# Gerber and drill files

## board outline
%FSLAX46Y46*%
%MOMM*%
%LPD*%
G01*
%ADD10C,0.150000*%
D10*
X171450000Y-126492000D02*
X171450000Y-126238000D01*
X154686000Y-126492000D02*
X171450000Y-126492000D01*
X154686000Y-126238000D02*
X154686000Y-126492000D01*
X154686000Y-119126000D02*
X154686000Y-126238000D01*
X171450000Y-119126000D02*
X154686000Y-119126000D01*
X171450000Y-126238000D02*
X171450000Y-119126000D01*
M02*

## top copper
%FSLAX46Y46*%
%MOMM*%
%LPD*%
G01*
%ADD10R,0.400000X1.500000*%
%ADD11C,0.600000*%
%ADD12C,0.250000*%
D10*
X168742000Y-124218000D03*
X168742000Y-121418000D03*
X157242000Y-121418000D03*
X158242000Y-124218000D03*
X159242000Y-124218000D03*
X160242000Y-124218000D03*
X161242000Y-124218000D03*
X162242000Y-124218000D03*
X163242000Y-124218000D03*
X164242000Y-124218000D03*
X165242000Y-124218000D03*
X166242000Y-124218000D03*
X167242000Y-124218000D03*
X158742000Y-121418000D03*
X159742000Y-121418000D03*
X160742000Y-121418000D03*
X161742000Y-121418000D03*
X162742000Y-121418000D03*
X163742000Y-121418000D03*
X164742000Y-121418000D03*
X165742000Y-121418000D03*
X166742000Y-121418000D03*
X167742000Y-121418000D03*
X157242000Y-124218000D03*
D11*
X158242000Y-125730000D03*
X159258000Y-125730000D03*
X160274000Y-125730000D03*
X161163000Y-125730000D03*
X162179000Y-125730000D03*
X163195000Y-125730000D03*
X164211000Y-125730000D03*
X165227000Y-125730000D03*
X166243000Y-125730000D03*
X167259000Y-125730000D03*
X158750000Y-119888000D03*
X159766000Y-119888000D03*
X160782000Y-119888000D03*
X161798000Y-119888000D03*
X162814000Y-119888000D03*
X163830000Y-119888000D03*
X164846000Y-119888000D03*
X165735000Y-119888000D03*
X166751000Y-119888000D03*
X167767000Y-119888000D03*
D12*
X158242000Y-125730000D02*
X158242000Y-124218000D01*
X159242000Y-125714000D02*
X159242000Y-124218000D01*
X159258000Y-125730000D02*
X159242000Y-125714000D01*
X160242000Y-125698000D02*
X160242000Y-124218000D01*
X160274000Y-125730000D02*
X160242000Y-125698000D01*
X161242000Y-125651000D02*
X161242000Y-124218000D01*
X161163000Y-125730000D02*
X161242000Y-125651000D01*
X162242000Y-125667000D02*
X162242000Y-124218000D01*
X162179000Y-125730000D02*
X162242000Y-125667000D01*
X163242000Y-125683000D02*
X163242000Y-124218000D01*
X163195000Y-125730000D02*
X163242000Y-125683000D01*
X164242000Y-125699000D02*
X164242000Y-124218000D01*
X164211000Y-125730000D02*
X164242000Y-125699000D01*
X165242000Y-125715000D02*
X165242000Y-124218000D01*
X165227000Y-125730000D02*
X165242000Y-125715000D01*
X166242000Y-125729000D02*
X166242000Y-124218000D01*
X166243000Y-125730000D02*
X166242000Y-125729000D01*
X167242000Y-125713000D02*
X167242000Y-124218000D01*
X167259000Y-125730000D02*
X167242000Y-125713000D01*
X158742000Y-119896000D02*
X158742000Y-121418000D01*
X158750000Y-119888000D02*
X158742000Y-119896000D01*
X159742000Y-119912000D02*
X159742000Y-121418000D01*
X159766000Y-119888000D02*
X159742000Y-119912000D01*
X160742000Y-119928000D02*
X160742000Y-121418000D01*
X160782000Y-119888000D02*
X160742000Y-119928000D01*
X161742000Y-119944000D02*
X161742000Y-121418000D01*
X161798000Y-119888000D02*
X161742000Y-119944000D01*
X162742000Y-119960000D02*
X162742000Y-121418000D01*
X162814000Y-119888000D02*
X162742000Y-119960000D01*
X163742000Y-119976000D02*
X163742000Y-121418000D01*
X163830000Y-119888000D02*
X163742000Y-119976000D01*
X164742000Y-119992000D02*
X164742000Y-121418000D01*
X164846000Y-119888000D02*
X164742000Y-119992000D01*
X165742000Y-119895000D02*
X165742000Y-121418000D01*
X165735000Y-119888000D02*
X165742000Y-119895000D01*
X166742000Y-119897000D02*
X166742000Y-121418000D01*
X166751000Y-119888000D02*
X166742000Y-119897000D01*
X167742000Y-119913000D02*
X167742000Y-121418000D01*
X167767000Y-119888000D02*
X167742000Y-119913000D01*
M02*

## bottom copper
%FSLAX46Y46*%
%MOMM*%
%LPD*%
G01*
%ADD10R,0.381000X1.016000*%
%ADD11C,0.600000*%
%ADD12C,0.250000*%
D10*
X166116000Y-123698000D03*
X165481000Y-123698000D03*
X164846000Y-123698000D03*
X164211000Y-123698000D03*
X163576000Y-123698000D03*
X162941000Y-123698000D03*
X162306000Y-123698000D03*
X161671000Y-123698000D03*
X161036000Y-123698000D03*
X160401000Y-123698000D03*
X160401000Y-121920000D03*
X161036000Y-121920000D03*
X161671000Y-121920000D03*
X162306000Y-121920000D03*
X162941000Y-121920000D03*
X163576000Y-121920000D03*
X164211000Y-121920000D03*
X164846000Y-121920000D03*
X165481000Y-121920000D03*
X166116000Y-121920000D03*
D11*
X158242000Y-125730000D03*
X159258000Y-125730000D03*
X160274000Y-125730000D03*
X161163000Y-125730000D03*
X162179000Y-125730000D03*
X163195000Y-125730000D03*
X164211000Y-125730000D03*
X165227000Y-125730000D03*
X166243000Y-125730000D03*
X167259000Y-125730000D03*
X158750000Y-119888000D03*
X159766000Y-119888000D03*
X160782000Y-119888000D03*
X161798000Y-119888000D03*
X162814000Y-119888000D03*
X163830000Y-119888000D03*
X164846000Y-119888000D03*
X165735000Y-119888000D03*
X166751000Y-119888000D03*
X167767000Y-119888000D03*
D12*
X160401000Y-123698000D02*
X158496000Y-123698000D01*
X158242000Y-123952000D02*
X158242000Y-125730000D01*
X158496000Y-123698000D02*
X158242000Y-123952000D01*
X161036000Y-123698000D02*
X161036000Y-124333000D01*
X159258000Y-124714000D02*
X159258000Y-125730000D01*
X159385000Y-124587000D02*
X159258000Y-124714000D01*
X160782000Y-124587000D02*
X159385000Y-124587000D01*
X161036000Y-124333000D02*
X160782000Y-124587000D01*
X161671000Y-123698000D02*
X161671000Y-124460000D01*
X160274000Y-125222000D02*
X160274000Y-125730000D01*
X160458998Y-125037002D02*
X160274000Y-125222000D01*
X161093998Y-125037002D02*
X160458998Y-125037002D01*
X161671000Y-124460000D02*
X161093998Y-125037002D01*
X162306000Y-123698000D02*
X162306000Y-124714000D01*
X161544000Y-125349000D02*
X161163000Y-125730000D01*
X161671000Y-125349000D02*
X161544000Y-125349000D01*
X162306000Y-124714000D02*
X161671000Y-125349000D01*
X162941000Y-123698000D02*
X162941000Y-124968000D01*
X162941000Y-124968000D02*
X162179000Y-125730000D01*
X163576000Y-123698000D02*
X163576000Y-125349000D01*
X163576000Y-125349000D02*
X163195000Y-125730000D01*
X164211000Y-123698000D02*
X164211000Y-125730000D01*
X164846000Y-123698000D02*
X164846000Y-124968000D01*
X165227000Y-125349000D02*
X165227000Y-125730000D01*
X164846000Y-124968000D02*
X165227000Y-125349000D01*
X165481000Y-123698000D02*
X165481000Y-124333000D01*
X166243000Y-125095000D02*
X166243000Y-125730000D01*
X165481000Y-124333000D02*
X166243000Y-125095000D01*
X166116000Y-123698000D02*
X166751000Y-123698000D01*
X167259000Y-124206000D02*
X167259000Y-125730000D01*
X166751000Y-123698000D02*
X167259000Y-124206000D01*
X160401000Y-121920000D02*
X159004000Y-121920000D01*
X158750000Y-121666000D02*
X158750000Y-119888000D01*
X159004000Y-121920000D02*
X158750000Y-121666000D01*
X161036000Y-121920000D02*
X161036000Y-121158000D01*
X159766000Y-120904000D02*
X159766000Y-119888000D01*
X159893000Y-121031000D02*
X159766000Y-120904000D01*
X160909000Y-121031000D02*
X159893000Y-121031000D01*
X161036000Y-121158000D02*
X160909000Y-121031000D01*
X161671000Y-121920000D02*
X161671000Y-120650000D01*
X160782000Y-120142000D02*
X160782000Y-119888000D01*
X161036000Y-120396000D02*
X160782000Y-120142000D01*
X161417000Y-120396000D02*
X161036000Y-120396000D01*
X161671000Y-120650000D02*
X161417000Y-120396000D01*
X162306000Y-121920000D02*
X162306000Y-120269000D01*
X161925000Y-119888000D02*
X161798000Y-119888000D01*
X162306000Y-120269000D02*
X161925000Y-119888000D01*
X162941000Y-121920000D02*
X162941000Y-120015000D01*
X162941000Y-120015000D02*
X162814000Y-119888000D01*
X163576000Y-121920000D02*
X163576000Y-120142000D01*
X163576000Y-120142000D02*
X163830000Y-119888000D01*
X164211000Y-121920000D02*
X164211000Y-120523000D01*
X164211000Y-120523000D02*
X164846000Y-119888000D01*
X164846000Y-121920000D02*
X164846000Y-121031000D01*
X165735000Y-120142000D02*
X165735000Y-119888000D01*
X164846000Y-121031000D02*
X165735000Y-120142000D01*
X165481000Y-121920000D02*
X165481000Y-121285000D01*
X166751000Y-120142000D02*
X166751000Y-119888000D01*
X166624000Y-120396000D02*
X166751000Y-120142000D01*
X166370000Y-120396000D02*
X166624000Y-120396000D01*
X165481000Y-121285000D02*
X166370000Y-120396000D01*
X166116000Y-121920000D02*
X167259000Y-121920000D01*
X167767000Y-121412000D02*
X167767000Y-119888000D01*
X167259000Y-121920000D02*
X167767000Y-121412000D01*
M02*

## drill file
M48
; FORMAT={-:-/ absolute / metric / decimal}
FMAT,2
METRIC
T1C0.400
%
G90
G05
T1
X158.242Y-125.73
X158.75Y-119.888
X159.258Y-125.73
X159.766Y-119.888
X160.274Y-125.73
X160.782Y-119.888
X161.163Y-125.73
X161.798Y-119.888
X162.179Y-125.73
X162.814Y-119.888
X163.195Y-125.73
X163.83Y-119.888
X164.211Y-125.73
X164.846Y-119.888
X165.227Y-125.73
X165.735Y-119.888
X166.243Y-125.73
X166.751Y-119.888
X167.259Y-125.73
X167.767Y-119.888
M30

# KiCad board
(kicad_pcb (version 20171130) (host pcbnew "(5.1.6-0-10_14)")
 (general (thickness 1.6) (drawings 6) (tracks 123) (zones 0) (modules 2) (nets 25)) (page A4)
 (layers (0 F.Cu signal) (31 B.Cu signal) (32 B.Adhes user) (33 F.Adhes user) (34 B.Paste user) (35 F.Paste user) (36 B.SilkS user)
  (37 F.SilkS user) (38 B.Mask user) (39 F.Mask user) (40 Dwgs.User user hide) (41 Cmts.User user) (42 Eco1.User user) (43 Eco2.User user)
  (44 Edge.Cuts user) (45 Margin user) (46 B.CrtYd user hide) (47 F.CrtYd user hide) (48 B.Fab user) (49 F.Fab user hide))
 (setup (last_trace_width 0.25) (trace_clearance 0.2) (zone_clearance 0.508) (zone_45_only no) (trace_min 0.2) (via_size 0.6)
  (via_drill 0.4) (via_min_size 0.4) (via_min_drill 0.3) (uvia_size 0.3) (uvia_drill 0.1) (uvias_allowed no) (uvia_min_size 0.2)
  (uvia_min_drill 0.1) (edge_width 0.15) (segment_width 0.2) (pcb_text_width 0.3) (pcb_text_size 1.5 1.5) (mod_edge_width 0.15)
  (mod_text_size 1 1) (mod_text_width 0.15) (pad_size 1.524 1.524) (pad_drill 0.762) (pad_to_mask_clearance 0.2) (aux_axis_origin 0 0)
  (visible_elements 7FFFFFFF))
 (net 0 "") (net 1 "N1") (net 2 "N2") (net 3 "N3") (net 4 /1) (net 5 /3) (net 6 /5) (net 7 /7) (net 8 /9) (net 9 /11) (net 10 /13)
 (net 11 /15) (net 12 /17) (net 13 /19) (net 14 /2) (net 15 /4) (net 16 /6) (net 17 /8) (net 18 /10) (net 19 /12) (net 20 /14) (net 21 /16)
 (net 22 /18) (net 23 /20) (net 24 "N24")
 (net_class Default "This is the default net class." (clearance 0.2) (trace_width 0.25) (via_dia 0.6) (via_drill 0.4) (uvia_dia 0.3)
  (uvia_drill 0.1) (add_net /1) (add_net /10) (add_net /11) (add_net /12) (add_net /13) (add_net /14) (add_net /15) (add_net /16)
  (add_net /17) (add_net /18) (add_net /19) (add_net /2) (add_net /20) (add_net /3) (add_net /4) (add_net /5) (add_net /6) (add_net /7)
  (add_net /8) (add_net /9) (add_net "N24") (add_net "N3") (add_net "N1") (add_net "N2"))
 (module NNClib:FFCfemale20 (layer F.Cu) (at 158.242 124.968)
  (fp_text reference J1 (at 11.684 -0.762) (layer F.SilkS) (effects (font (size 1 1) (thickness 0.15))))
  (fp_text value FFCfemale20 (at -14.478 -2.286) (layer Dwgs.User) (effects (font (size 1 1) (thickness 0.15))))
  (pad 42 smd rect (at 10.5 -0.75) (size 0.4 1.5) (layers F.Cu F.Paste F.Mask) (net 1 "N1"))
  (pad 43 smd rect (at 10.5 -3.55) (size 0.4 1.5) (layers F.Cu F.Paste F.Mask) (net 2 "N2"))
  (pad 41 smd rect (at -1 -3.55) (size 0.4 1.5) (layers F.Cu F.Paste F.Mask) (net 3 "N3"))
  (pad 1 smd rect (at 0 -0.75 180) (size 0.4 1.5) (layers F.Cu F.Paste F.Mask) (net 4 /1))
  (pad 3 smd rect (at 1 -0.75 180) (size 0.4 1.5) (layers F.Cu F.Paste F.Mask) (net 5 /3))
  (pad 5 smd rect (at 2 -0.75 180) (size 0.4 1.5) (layers F.Cu F.Paste F.Mask) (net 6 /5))
  (pad 7 smd rect (at 3 -0.75 180) (size 0.4 1.5) (layers F.Cu F.Paste F.Mask) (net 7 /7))
  (pad 9 smd rect (at 4 -0.75 180) (size 0.4 1.5) (layers F.Cu F.Paste F.Mask) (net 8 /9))
  (pad 11 smd rect (at 5 -0.75 180) (size 0.4 1.5) (layers F.Cu F.Paste F.Mask) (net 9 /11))
  (pad 13 smd rect (at 6 -0.75 180) (size 0.4 1.5) (layers F.Cu F.Paste F.Mask) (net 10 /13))
  (pad 15 smd rect (at 7 -0.75 180) (size 0.4 1.5) (layers F.Cu F.Paste F.Mask) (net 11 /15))
  (pad 17 smd rect (at 8 -0.75 180) (size 0.4 1.5) (layers F.Cu F.Paste F.Mask) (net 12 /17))
  (pad 19 smd rect (at 9 -0.75 180) (size 0.4 1.5) (layers F.Cu F.Paste F.Mask) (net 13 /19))
  (pad 2 smd rect (at 0.5 -3.55 180) (size 0.4 1.5) (layers F.Cu F.Paste F.Mask) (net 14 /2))
  (pad 4 smd rect (at 1.5 -3.55 180) (size 0.4 1.5) (layers F.Cu F.Paste F.Mask) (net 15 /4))
  (pad 6 smd rect (at 2.5 -3.55 180) (size 0.4 1.5) (layers F.Cu F.Paste F.Mask) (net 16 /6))
  (pad 8 smd rect (at 3.5 -3.55 180) (size 0.4 1.5) (layers F.Cu F.Paste F.Mask) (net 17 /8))
  (pad 10 smd rect (at 4.5 -3.55 180) (size 0.4 1.5) (layers F.Cu F.Paste F.Mask) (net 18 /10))
  (pad 12 smd rect (at 5.5 -3.55 180) (size 0.4 1.5) (layers F.Cu F.Paste F.Mask) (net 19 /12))
  (pad 14 smd rect (at 6.5 -3.55 180) (size 0.4 1.5) (layers F.Cu F.Paste F.Mask) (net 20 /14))
  (pad 16 smd rect (at 7.5 -3.55 180) (size 0.4 1.5) (layers F.Cu F.Paste F.Mask) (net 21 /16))
  (pad 18 smd rect (at 8.5 -3.55 180) (size 0.4 1.5) (layers F.Cu F.Paste F.Mask) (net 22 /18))
  (pad 20 smd rect (at 9.5 -3.55 180) (size 0.4 1.5) (layers F.Cu F.Paste F.Mask) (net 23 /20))
  (pad 40 smd rect (at -1 -0.75) (size 0.4 1.5) (layers F.Cu F.Paste F.Mask) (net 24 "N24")))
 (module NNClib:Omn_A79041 (layer B.Cu) (at 160.401 121.412)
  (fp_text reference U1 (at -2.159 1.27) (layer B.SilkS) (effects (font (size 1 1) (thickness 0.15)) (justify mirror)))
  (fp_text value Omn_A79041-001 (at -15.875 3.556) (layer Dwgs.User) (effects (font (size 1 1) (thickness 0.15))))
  (pad 20 smd rect (at 5.715 2.286 180) (size 0.381 1.016) (layers B.Cu B.Paste B.Mask) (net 13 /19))
  (pad 18 smd rect (at 5.08 2.286 180) (size 0.381 1.016) (layers B.Cu B.Paste B.Mask) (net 12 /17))
  (pad 16 smd rect (at 4.445 2.286 180) (size 0.381 1.016) (layers B.Cu B.Paste B.Mask) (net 11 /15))
  (pad 14 smd rect (at 3.81 2.286 180) (size 0.381 1.016) (layers B.Cu B.Paste B.Mask) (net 10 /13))
  (pad 12 smd rect (at 3.175 2.286 180) (size 0.381 1.016) (layers B.Cu B.Paste B.Mask) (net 9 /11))
  (pad 10 smd rect (at 2.54 2.286 180) (size 0.381 1.016) (layers B.Cu B.Paste B.Mask) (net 8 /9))
  (pad 8 smd rect (at 1.905 2.286 180) (size 0.381 1.016) (layers B.Cu B.Paste B.Mask) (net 7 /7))
  (pad 6 smd rect (at 1.27 2.286 180) (size 0.381 1.016) (layers B.Cu B.Paste B.Mask) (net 6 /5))
  (pad 4 smd rect (at 0.635 2.286 180) (size 0.381 1.016) (layers B.Cu B.Paste B.Mask) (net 5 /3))
  (pad 2 smd rect (at 0 2.286 180) (size 0.381 1.016) (layers B.Cu B.Paste B.Mask) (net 4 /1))
  (pad 1 smd rect (at 0 0.508 180) (size 0.381 1.016) (layers B.Cu B.Paste B.Mask) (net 14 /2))
  (pad 3 smd rect (at 0.635 0.508 180) (size 0.381 1.016) (layers B.Cu B.Paste B.Mask) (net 15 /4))
  (pad 5 smd rect (at 1.27 0.508 180) (size 0.381 1.016) (layers B.Cu B.Paste B.Mask) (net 16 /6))
  (pad 7 smd rect (at 1.905 0.508 180) (size 0.381 1.016) (layers B.Cu B.Paste B.Mask) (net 17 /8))
  (pad 9 smd rect (at 2.54 0.508 180) (size 0.381 1.016) (layers B.Cu B.Paste B.Mask) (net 18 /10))
  (pad 11 smd rect (at 3.175 0.508 180) (size 0.381 1.016) (layers B.Cu B.Paste B.Mask) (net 19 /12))
  (pad 13 smd rect (at 3.81 0.508 180) (size 0.381 1.016) (layers B.Cu B.Paste B.Mask) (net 20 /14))
  (pad 15 smd rect (at 4.445 0.508 180) (size 0.381 1.016) (layers B.Cu B.Paste B.Mask) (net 21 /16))
  (pad 17 smd rect (at 5.08 0.508 180) (size 0.381 1.016) (layers B.Cu B.Paste B.Mask) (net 22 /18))
  (pad 19 smd rect (at 5.715 0.508 180) (size 0.381 1.016) (layers B.Cu B.Paste B.Mask) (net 23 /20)))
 (gr_line (start 171.45 126.492) (end 171.45 126.238) (angle 90) (layer Edge.Cuts) (width 0.15))
 (gr_line (start 154.686 126.492) (end 171.45 126.492) (angle 90) (layer Edge.Cuts) (width 0.15))
 (gr_line (start 154.686 126.238) (end 154.686 126.492) (angle 90) (layer Edge.Cuts) (width 0.15))
 (gr_line (start 154.686 119.126) (end 154.686 126.238) (angle 90) (layer Edge.Cuts) (width 0.15))
 (gr_line (start 171.45 119.126) (end 154.686 119.126) (angle 90) (layer Edge.Cuts) (width 0.15))
 (gr_line (start 171.45 126.238) (end 171.45 119.126) (angle 90) (layer Edge.Cuts) (width 0.15))
 (segment (start 160.401 123.698) (end 158.496 123.698) (width 0.25) (layer B.Cu) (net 4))
 (segment (start 158.242 125.73) (end 158.242 124.218) (width 0.25) (layer F.Cu) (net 4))
 (via (at 158.242 125.73) (size 0.6) (drill 0.4) (layers F.Cu B.Cu) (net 4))
 (segment (start 158.242 123.952) (end 158.242 125.73) (width 0.25) (layer B.Cu) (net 4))
 (segment (start 158.496 123.698) (end 158.242 123.952) (width 0.25) (layer B.Cu) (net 4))
 (segment (start 161.036 123.698) (end 161.036 124.333) (width 0.25) (layer B.Cu) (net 5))
 (segment (start 159.242 125.714) (end 159.242 124.218) (width 0.25) (layer F.Cu) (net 5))
 (segment (start 159.258 125.73) (end 159.242 125.714) (width 0.25) (layer F.Cu) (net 5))
 (via (at 159.258 125.73) (size 0.6) (drill 0.4) (layers F.Cu B.Cu) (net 5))
 (segment (start 159.258 124.714) (end 159.258 125.73) (width 0.25) (layer B.Cu) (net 5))
 (segment (start 159.385 124.587) (end 159.258 124.714) (width 0.25) (layer B.Cu) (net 5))
 (segment (start 160.782 124.587) (end 159.385 124.587) (width 0.25) (layer B.Cu) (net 5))
 (segment (start 161.036 124.333) (end 160.782 124.587) (width 0.25) (layer B.Cu) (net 5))
 (segment (start 161.671 123.698) (end 161.671 124.46) (width 0.25) (layer B.Cu) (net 6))
 (segment (start 160.242 125.698) (end 160.242 124.218) (width 0.25) (layer F.Cu) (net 6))
 (segment (start 160.274 125.73) (end 160.242 125.698) (width 0.25) (layer F.Cu) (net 6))
 (via (at 160.274 125.73) (size 0.6) (drill 0.4) (layers F.Cu B.Cu) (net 6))
 (segment (start 160.274 125.222) (end 160.274 125.73) (width 0.25) (layer B.Cu) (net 6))
 (segment (start 160.458998 125.037002) (end 160.274 125.222) (width 0.25) (layer B.Cu) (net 6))
 (segment (start 161.093998 125.037002) (end 160.458998 125.037002) (width 0.25) (layer B.Cu) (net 6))
 (segment (start 161.671 124.46) (end 161.093998 125.037002) (width 0.25) (layer B.Cu) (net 6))
 (segment (start 162.306 123.698) (end 162.306 124.714) (width 0.25) (layer B.Cu) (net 7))
 (segment (start 161.242 125.651) (end 161.242 124.218) (width 0.25) (layer F.Cu) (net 7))
 (segment (start 161.163 125.73) (end 161.242 125.651) (width 0.25) (layer F.Cu) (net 7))
 (via (at 161.163 125.73) (size 0.6) (drill 0.4) (layers F.Cu B.Cu) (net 7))
 (segment (start 161.544 125.349) (end 161.163 125.73) (width 0.25) (layer B.Cu) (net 7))
 (segment (start 161.671 125.349) (end 161.544 125.349) (width 0.25) (layer B.Cu) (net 7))
 (segment (start 162.306 124.714) (end 161.671 125.349) (width 0.25) (layer B.Cu) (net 7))
 (segment (start 162.941 123.698) (end 162.941 124.968) (width 0.25) (layer B.Cu) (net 8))
 (segment (start 162.242 125.667) (end 162.242 124.218) (width 0.25) (layer F.Cu) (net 8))
 (segment (start 162.179 125.73) (end 162.242 125.667) (width 0.25) (layer F.Cu) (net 8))
 (via (at 162.179 125.73) (size 0.6) (drill 0.4) (layers F.Cu B.Cu) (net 8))
 (segment (start 162.941 124.968) (end 162.179 125.73) (width 0.25) (layer B.Cu) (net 8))
 (segment (start 163.576 123.698) (end 163.576 125.349) (width 0.25) (layer B.Cu) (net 9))
 (segment (start 163.242 125.683) (end 163.242 124.218) (width 0.25) (layer F.Cu) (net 9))
 (segment (start 163.195 125.73) (end 163.242 125.683) (width 0.25) (layer F.Cu) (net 9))
 (via (at 163.195 125.73) (size 0.6) (drill 0.4) (layers F.Cu B.Cu) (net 9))
 (segment (start 163.576 125.349) (end 163.195 125.73) (width 0.25) (layer B.Cu) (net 9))
 (segment (start 164.211 123.698) (end 164.211 125.73) (width 0.25) (layer B.Cu) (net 10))
 (segment (start 164.242 125.699) (end 164.242 124.218) (width 0.25) (layer F.Cu) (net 10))
 (segment (start 164.211 125.73) (end 164.242 125.699) (width 0.25) (layer F.Cu) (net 10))
 (via (at 164.211 125.73) (size 0.6) (drill 0.4) (layers F.Cu B.Cu) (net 10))
 (segment (start 164.846 123.698) (end 164.846 124.968) (width 0.25) (layer B.Cu) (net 11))
 (segment (start 165.242 125.715) (end 165.242 124.218) (width 0.25) (layer F.Cu) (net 11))
 (segment (start 165.227 125.73) (end 165.242 125.715) (width 0.25) (layer F.Cu) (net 11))
 (via (at 165.227 125.73) (size 0.6) (drill 0.4) (layers F.Cu B.Cu) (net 11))
 (segment (start 165.227 125.349) (end 165.227 125.73) (width 0.25) (layer B.Cu) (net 11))
 (segment (start 164.846 124.968) (end 165.227 125.349) (width 0.25) (layer B.Cu) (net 11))
 (segment (start 165.481 123.698) (end 165.481 124.333) (width 0.25) (layer B.Cu) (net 12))
 (segment (start 166.242 125.729) (end 166.242 124.218) (width 0.25) (layer F.Cu) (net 12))
 (segment (start 166.243 125.73) (end 166.242 125.729) (width 0.25) (layer F.Cu) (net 12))
 (via (at 166.243 125.73) (size 0.6) (drill 0.4) (layers F.Cu B.Cu) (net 12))
 (segment (start 166.243 125.095) (end 166.243 125.73) (width 0.25) (layer B.Cu) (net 12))
 (segment (start 165.481 124.333) (end 166.243 125.095) (width 0.25) (layer B.Cu) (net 12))
 (segment (start 166.116 123.698) (end 166.751 123.698) (width 0.25) (layer B.Cu) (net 13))
 (segment (start 167.242 125.713) (end 167.242 124.218) (width 0.25) (layer F.Cu) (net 13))
 (segment (start 167.259 125.73) (end 167.242 125.713) (width 0.25) (layer F.Cu) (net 13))
 (via (at 167.259 125.73) (size 0.6) (drill 0.4) (layers F.Cu B.Cu) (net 13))
 (segment (start 167.259 124.206) (end 167.259 125.73) (width 0.25) (layer B.Cu) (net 13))
 (segment (start 166.751 123.698) (end 167.259 124.206) (width 0.25) (layer B.Cu) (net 13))
 (segment (start 160.401 121.92) (end 159.004 121.92) (width 0.25) (layer B.Cu) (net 14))
 (segment (start 158.742 119.896) (end 158.742 121.418) (width 0.25) (layer F.Cu) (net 14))
 (segment (start 158.75 119.888) (end 158.742 119.896) (width 0.25) (layer F.Cu) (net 14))
 (via (at 158.75 119.888) (size 0.6) (drill 0.4) (layers F.Cu B.Cu) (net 14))
 (segment (start 158.75 121.666) (end 158.75 119.888) (width 0.25) (layer B.Cu) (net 14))
 (segment (start 159.004 121.92) (end 158.75 121.666) (width 0.25) (layer B.Cu) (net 14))
 (segment (start 161.036 121.92) (end 161.036 121.158) (width 0.25) (layer B.Cu) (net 15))
 (segment (start 159.742 119.912) (end 159.742 121.418) (width 0.25) (layer F.Cu) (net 15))
 (segment (start 159.766 119.888) (end 159.742 119.912) (width 0.25) (layer F.Cu) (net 15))
 (via (at 159.766 119.888) (size 0.6) (drill 0.4) (layers F.Cu B.Cu) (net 15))
 (segment (start 159.766 120.904) (end 159.766 119.888) (width 0.25) (layer B.Cu) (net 15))
 (segment (start 159.893 121.031) (end 159.766 120.904) (width 0.25) (layer B.Cu) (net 15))
 (segment (start 160.909 121.031) (end 159.893 121.031) (width 0.25) (layer B.Cu) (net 15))
 (segment (start 161.036 121.158) (end 160.909 121.031) (width 0.25) (layer B.Cu) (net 15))
 (segment (start 161.671 121.92) (end 161.671 120.65) (width 0.25) (layer B.Cu) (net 16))
 (segment (start 160.742 119.928) (end 160.742 121.418) (width 0.25) (layer F.Cu) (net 16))
 (segment (start 160.782 119.888) (end 160.742 119.928) (width 0.25) (layer F.Cu) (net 16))
 (via (at 160.782 119.888) (size 0.6) (drill 0.4) (layers F.Cu B.Cu) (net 16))
 (segment (start 160.782 120.142) (end 160.782 119.888) (width 0.25) (layer B.Cu) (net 16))
 (segment (start 161.036 120.396) (end 160.782 120.142) (width 0.25) (layer B.Cu) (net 16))
 (segment (start 161.417 120.396) (end 161.036 120.396) (width 0.25) (layer B.Cu) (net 16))
 (segment (start 161.671 120.65) (end 161.417 120.396) (width 0.25) (layer B.Cu) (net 16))
 (segment (start 162.306 121.92) (end 162.306 120.269) (width 0.25) (layer B.Cu) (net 17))
 (segment (start 161.742 119.944) (end 161.742 121.418) (width 0.25) (layer F.Cu) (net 17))
 (segment (start 161.798 119.888) (end 161.742 119.944) (width 0.25) (layer F.Cu) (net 17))
 (via (at 161.798 119.888) (size 0.6) (drill 0.4) (layers F.Cu B.Cu) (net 17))
 (segment (start 161.925 119.888) (end 161.798 119.888) (width 0.25) (layer B.Cu) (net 17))
 (segment (start 162.306 120.269) (end 161.925 119.888) (width 0.25) (layer B.Cu) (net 17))
 (segment (start 162.941 121.92) (end 162.941 120.015) (width 0.25) (layer B.Cu) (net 18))
 (segment (start 162.742 119.96) (end 162.742 121.418) (width 0.25) (layer F.Cu) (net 18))
 (segment (start 162.814 119.888) (end 162.742 119.96) (width 0.25) (layer F.Cu) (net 18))
 (via (at 162.814 119.888) (size 0.6) (drill 0.4) (layers F.Cu B.Cu) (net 18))
 (segment (start 162.941 120.015) (end 162.814 119.888) (width 0.25) (layer B.Cu) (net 18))
 (segment (start 163.576 121.92) (end 163.576 120.142) (width 0.25) (layer B.Cu) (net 19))
 (segment (start 163.742 119.976) (end 163.742 121.418) (width 0.25) (layer F.Cu) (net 19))
 (segment (start 163.83 119.888) (end 163.742 119.976) (width 0.25) (layer F.Cu) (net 19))
 (via (at 163.83 119.888) (size 0.6) (drill 0.4) (layers F.Cu B.Cu) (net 19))
 (segment (start 163.576 120.142) (end 163.83 119.888) (width 0.25) (layer B.Cu) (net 19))
 (segment (start 164.211 121.92) (end 164.211 120.523) (width 0.25) (layer B.Cu) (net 20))
 (segment (start 164.742 119.992) (end 164.742 121.418) (width 0.25) (layer F.Cu) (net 20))
 (segment (start 164.846 119.888) (end 164.742 119.992) (width 0.25) (layer F.Cu) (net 20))
 (via (at 164.846 119.888) (size 0.6) (drill 0.4) (layers F.Cu B.Cu) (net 20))
 (segment (start 164.211 120.523) (end 164.846 119.888) (width 0.25) (layer B.Cu) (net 20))
 (segment (start 164.846 121.92) (end 164.846 121.031) (width 0.25) (layer B.Cu) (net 21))
 (segment (start 165.742 119.895) (end 165.742 121.418) (width 0.25) (layer F.Cu) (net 21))
 (segment (start 165.735 119.888) (end 165.742 119.895) (width 0.25) (layer F.Cu) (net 21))
 (via (at 165.735 119.888) (size 0.6) (drill 0.4) (layers F.Cu B.Cu) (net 21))
 (segment (start 165.735 120.142) (end 165.735 119.888) (width 0.25) (layer B.Cu) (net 21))
 (segment (start 164.846 121.031) (end 165.735 120.142) (width 0.25) (layer B.Cu) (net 21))
 (segment (start 165.481 121.92) (end 165.481 121.285) (width 0.25) (layer B.Cu) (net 22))
 (segment (start 166.742 119.897) (end 166.742 121.418) (width 0.25) (layer F.Cu) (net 22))
 (segment (start 166.751 119.888) (end 166.742 119.897) (width 0.25) (layer F.Cu) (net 22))
 (via (at 166.751 119.888) (size 0.6) (drill 0.4) (layers F.Cu B.Cu) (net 22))
 (segment (start 166.751 120.142) (end 166.751 119.888) (width 0.25) (layer B.Cu) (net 22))
 (segment (start 166.624 120.396) (end 166.751 120.142) (width 0.25) (layer B.Cu) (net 22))
 (segment (start 166.37 120.396) (end 166.624 120.396) (width 0.25) (layer B.Cu) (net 22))
 (segment (start 165.481 121.285) (end 166.37 120.396) (width 0.25) (layer B.Cu) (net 22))
 (segment (start 166.116 121.92) (end 167.259 121.92) (width 0.25) (layer B.Cu) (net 23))
 (segment (start 167.742 119.913) (end 167.742 121.418) (width 0.25) (layer F.Cu) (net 23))
 (segment (start 167.767 119.888) (end 167.742 119.913) (width 0.25) (layer F.Cu) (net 23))
 (via (at 167.767 119.888) (size 0.6) (drill 0.4) (layers F.Cu B.Cu) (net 23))
 (segment (start 167.767 121.412) (end 167.767 119.888) (width 0.25) (layer B.Cu) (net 23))
 (segment (start 167.259 121.92) (end 167.767 121.412) (width 0.25) (layer B.Cu) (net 23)))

